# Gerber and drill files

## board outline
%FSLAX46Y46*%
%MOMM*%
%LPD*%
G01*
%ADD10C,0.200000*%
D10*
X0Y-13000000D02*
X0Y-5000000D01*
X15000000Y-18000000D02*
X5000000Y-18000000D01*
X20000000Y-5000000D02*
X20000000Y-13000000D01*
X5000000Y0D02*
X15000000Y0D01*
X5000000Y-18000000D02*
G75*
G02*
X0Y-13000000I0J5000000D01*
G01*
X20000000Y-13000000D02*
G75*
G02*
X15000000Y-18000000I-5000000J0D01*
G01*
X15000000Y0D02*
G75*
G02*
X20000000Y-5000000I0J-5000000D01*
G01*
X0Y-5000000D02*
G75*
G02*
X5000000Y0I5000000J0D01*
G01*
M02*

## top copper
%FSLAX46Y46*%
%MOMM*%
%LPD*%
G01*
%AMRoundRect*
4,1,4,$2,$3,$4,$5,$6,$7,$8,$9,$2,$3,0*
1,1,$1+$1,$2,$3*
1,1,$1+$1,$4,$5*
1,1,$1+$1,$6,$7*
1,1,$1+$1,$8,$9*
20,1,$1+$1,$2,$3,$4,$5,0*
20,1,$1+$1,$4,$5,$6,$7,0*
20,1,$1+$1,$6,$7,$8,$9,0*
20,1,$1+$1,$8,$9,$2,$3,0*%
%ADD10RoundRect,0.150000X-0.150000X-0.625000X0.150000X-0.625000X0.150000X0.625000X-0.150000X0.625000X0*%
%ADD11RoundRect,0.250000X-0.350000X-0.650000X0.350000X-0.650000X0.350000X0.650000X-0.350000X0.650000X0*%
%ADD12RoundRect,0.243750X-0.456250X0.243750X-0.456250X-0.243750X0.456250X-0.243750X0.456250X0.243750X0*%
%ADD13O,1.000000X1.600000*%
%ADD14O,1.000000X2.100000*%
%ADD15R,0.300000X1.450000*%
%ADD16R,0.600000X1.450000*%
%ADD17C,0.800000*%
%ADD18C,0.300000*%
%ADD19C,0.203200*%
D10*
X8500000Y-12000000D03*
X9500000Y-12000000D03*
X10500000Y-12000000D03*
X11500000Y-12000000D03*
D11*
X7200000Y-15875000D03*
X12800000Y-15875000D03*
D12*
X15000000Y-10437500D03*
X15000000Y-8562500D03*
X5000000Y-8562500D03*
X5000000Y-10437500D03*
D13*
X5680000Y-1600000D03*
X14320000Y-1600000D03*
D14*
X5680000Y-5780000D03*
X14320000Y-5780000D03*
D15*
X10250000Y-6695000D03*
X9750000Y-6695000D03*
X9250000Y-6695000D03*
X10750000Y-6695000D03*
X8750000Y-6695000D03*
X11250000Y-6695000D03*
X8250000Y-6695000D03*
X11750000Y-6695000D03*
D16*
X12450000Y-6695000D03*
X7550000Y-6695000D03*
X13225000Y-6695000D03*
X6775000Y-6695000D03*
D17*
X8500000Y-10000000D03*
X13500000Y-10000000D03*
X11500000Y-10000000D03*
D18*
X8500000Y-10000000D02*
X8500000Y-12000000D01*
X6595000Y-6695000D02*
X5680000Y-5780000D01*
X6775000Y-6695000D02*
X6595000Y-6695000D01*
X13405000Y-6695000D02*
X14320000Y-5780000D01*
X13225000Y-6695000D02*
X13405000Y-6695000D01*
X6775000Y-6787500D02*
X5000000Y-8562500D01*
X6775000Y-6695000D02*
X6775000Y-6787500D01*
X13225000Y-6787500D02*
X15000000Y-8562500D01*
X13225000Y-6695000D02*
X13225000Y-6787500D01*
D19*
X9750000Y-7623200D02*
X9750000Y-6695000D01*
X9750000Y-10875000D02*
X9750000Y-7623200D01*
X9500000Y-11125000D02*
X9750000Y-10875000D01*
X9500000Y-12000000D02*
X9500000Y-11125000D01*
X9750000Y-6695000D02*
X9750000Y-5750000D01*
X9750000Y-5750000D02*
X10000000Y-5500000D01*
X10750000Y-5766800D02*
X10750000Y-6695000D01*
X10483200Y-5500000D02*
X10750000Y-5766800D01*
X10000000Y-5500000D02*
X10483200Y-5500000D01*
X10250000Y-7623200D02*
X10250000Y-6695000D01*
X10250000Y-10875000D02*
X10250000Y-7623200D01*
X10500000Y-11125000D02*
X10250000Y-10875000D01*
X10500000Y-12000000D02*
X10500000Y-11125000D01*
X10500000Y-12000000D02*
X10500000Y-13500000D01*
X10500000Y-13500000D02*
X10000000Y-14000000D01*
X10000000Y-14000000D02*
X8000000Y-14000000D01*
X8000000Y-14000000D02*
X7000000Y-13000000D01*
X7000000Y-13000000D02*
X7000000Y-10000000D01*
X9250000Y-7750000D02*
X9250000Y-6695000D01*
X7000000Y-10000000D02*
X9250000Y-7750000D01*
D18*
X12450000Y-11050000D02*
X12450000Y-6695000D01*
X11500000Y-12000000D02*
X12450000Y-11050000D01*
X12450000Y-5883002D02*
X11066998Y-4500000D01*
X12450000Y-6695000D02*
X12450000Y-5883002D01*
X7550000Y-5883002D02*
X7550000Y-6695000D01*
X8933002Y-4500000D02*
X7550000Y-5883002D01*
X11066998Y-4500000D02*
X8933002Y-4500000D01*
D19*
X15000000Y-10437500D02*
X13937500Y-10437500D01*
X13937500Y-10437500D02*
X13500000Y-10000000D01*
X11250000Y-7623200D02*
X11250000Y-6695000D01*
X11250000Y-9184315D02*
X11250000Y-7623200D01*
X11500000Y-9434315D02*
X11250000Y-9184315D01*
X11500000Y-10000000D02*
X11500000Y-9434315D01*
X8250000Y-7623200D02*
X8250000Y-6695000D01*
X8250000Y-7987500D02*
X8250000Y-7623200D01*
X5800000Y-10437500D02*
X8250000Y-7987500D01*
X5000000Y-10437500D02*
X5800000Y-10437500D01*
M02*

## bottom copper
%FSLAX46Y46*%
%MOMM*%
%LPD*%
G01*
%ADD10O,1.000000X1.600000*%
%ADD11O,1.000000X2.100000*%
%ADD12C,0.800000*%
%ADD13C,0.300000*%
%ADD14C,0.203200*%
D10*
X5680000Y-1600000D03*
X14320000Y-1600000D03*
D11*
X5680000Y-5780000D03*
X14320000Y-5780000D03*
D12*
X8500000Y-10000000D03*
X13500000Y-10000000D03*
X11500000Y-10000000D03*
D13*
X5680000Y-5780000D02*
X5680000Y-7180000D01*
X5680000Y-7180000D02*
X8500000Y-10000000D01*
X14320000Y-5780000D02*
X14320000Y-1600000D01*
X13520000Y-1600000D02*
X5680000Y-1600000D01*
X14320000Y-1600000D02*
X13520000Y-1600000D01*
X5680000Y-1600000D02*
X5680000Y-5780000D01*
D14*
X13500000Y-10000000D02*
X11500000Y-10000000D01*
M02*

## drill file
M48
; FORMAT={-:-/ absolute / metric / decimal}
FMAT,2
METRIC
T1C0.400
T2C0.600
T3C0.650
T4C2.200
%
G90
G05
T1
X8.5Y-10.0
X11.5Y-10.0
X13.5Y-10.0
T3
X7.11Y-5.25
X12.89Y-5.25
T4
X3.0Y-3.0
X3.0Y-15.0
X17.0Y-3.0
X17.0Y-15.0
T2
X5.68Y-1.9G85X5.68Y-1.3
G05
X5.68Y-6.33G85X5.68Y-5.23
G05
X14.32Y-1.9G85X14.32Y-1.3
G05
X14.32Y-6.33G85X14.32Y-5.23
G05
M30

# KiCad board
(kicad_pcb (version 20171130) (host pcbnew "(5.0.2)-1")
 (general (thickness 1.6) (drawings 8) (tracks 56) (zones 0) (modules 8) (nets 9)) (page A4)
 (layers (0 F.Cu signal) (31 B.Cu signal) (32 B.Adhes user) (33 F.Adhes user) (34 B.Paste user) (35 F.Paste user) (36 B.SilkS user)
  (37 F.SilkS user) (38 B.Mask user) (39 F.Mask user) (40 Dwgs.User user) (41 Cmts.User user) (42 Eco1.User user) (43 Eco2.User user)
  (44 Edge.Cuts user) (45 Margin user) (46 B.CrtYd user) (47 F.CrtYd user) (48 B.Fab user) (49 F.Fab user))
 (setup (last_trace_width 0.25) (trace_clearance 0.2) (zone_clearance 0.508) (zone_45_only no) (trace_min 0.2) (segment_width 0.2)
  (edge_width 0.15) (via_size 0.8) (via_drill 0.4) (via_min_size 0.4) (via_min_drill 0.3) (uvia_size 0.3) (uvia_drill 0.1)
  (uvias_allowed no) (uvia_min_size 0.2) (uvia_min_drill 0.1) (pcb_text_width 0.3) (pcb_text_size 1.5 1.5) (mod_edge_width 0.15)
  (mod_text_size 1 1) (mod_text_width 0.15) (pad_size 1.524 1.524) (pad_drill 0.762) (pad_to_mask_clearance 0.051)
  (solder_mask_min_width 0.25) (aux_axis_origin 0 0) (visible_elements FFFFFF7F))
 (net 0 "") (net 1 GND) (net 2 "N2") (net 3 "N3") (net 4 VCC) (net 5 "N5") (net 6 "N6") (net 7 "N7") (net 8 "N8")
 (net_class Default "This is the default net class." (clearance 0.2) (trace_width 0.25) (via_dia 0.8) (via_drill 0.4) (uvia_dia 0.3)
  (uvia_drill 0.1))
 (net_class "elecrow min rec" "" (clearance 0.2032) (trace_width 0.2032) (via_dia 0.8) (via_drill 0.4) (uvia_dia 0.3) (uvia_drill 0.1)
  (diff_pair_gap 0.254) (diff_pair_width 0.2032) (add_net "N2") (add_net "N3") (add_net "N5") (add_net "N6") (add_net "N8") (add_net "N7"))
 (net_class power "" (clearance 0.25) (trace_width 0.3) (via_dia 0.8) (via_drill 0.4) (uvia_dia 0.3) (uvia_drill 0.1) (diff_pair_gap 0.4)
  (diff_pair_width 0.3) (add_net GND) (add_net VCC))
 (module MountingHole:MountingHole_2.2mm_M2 (layer F.Cu) (at 3 15)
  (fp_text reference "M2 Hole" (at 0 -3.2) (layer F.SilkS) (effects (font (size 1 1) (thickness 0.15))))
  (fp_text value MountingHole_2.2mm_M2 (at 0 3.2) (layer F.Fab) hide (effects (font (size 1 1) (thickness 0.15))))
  (pad 1 np_thru_hole circle (at 0 0) (size 2.2 2.2) (drill 2.2) (layers *.Cu *.Mask)))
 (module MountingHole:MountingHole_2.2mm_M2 (layer F.Cu) (at 17 15)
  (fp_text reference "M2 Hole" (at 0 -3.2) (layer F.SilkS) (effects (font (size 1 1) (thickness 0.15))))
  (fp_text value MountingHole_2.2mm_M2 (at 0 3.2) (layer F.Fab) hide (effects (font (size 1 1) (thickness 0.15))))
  (pad 1 np_thru_hole circle (at 0 0) (size 2.2 2.2) (drill 2.2) (layers *.Cu *.Mask)))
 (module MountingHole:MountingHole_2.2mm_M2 (layer F.Cu) (at 17 3)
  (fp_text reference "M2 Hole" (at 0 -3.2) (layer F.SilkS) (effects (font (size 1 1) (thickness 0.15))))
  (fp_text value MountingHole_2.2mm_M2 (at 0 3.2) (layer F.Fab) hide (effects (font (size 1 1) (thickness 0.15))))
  (pad 1 np_thru_hole circle (at 0 0) (size 2.2 2.2) (drill 2.2) (layers *.Cu *.Mask)))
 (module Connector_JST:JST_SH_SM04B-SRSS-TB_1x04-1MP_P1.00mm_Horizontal (layer F.Cu) (at 10 14)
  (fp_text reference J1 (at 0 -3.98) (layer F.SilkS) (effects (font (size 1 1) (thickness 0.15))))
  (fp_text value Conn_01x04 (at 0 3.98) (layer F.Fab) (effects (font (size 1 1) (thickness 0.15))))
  (pad 1 smd roundrect (at -1.5 -2) (size 0.6 1.55) (layers F.Cu F.Paste F.Mask) (roundrect_rratio 0.25) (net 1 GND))
  (pad 2 smd roundrect (at -0.5 -2) (size 0.6 1.55) (layers F.Cu F.Paste F.Mask) (roundrect_rratio 0.25) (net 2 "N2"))
  (pad 3 smd roundrect (at 0.5 -2) (size 0.6 1.55) (layers F.Cu F.Paste F.Mask) (roundrect_rratio 0.25) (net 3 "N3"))
  (pad 4 smd roundrect (at 1.5 -2) (size 0.6 1.55) (layers F.Cu F.Paste F.Mask) (roundrect_rratio 0.25) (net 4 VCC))
  (pad MP smd roundrect (at -2.8 1.875) (size 1.2 1.8) (layers F.Cu F.Paste F.Mask) (roundrect_rratio 0.208333))
  (pad MP smd roundrect (at 2.8 1.875) (size 1.2 1.8) (layers F.Cu F.Paste F.Mask) (roundrect_rratio 0.208333)))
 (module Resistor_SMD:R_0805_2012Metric (layer F.Cu) (at 15 9.5 270)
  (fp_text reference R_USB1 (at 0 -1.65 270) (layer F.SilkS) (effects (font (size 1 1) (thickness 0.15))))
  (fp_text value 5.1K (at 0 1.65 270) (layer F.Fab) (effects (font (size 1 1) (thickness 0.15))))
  (pad 2 smd roundrect (at 0.9375 0 270) (size 0.975 1.4) (layers F.Cu F.Paste F.Mask) (roundrect_rratio 0.25) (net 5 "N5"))
  (pad 1 smd roundrect (at -0.9375 0 270) (size 0.975 1.4) (layers F.Cu F.Paste F.Mask) (roundrect_rratio 0.25) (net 1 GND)))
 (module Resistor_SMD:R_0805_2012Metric (layer F.Cu) (at 5 9.5 270)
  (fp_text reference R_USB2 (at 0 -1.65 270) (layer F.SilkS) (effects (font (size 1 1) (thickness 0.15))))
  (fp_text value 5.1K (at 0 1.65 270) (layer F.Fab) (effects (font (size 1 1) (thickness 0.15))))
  (pad 1 smd roundrect (at -0.9375 0 270) (size 0.975 1.4) (layers F.Cu F.Paste F.Mask) (roundrect_rratio 0.25) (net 1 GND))
  (pad 2 smd roundrect (at 0.9375 0 270) (size 0.975 1.4) (layers F.Cu F.Paste F.Mask) (roundrect_rratio 0.25) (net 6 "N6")))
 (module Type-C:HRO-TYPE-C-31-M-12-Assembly (layer F.Cu) (at 10 -1 180)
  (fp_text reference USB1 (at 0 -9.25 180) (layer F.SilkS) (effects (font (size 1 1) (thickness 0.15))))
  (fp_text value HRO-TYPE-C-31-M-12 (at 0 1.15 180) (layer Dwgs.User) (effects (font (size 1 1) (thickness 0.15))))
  (pad 13 thru_hole oval (at 4.32 -2.6 180) (size 1 1.6) (drill oval 0.6 1.2) (layers *.Cu *.Mask) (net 1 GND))
  (pad 13 thru_hole oval (at -4.32 -2.6 180) (size 1 1.6) (drill oval 0.6 1.2) (layers *.Cu *.Mask) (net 1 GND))
  (pad 13 thru_hole oval (at 4.32 -6.78 180) (size 1 2.1) (drill oval 0.6 1.7) (layers *.Cu *.Mask) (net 1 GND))
  (pad 13 thru_hole oval (at -4.32 -6.78 180) (size 1 2.1) (drill oval 0.6 1.7) (layers *.Cu *.Mask) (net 1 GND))
  (pad "" np_thru_hole circle (at -2.89 -6.25 180) (size 0.65 0.65) (drill 0.65) (layers *.Cu *.Mask))
  (pad "" np_thru_hole circle (at 2.89 -6.25 180) (size 0.65 0.65) (drill 0.65) (layers *.Cu *.Mask))
  (pad 6 smd rect (at -0.25 -7.695 180) (size 0.3 1.45) (layers F.Cu F.Paste F.Mask) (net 3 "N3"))
  (pad 7 smd rect (at 0.25 -7.695 180) (size 0.3 1.45) (layers F.Cu F.Paste F.Mask) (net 2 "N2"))
  (pad 8 smd rect (at 0.75 -7.695 180) (size 0.3 1.45) (layers F.Cu F.Paste F.Mask) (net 3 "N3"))
  (pad 5 smd rect (at -0.75 -7.695 180) (size 0.3 1.45) (layers F.Cu F.Paste F.Mask) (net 2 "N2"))
  (pad 9 smd rect (at 1.25 -7.695 180) (size 0.3 1.45) (layers F.Cu F.Paste F.Mask) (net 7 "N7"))
  (pad 4 smd rect (at -1.25 -7.695 180) (size 0.3 1.45) (layers F.Cu F.Paste F.Mask) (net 5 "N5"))
  (pad 10 smd rect (at 1.75 -7.695 180) (size 0.3 1.45) (layers F.Cu F.Paste F.Mask) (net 6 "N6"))
  (pad 3 smd rect (at -1.75 -7.695 180) (size 0.3 1.45) (layers F.Cu F.Paste F.Mask) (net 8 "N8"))
  (pad 2 smd rect (at -2.45 -7.695 180) (size 0.6 1.45) (layers F.Cu F.Paste F.Mask) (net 4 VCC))
  (pad 11 smd rect (at 2.45 -7.695 180) (size 0.6 1.45) (layers F.Cu F.Paste F.Mask) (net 4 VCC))
  (pad 1 smd rect (at -3.225 -7.695 180) (size 0.6 1.45) (layers F.Cu F.Paste F.Mask) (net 1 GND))
  (pad 12 smd rect (at 3.225 -7.695 180) (size 0.6 1.45) (layers F.Cu F.Paste F.Mask) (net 1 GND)))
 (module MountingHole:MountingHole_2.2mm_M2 (layer F.Cu) (at 3 3)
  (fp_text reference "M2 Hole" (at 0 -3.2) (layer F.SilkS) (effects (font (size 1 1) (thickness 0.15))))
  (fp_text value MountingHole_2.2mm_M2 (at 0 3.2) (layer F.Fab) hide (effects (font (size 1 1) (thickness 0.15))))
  (pad 1 np_thru_hole circle (at 0 0) (size 2.2 2.2) (drill 2.2) (layers *.Cu *.Mask)))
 (gr_line (start 0 13) (end 0 5) (layer Edge.Cuts) (width 0.2))
 (gr_line (start 15 18) (end 5 18) (layer Edge.Cuts) (width 0.2))
 (gr_line (start 20 5) (end 20 13) (layer Edge.Cuts) (width 0.2))
 (gr_line (start 5 0) (end 15 0) (layer Edge.Cuts) (width 0.2))
 (gr_arc (start 5 13) (end 0 13) (angle -90) (layer Edge.Cuts) (width 0.2))
 (gr_arc (start 15 13) (end 15 18) (angle -90) (layer Edge.Cuts) (width 0.2))
 (gr_arc (start 15 5) (end 20 5) (angle -90) (layer Edge.Cuts) (width 0.2))
 (gr_arc (start 5 5) (end 5 0) (angle -90) (layer Edge.Cuts) (width 0.2))
 (via (at 8.5 10) (size 0.8) (drill 0.4) (layers F.Cu B.Cu) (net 1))
 (segment (start 5.68 5.78) (end 5.68 7.18) (width 0.3) (layer B.Cu) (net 1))
 (segment (start 5.68 7.18) (end 8.5 10) (width 0.3) (layer B.Cu) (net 1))
 (segment (start 8.5 10) (end 8.5 12) (width 0.3) (layer F.Cu) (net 1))
 (segment (start 6.595 6.695) (end 5.68 5.78) (width 0.3) (layer F.Cu) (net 1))
 (segment (start 6.775 6.695) (end 6.595 6.695) (width 0.3) (layer F.Cu) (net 1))
 (segment (start 13.405 6.695) (end 14.32 5.78) (width 0.3) (layer F.Cu) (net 1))
 (segment (start 13.225 6.695) (end 13.405 6.695) (width 0.3) (layer F.Cu) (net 1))
 (segment (start 14.32 5.78) (end 14.32 1.6) (width 0.3) (layer B.Cu) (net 1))
 (segment (start 13.52 1.6) (end 5.68 1.6) (width 0.3) (layer B.Cu) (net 1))
 (segment (start 14.32 1.6) (end 13.52 1.6) (width 0.3) (layer B.Cu) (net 1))
 (segment (start 5.68 1.6) (end 5.68 5.78) (width 0.3) (layer B.Cu) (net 1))
 (segment (start 6.775 6.7875) (end 5 8.5625) (width 0.3) (layer F.Cu) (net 1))
 (segment (start 6.775 6.695) (end 6.775 6.7875) (width 0.3) (layer F.Cu) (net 1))
 (segment (start 13.225 6.7875) (end 15 8.5625) (width 0.3) (layer F.Cu) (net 1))
 (segment (start 13.225 6.695) (end 13.225 6.7875) (width 0.3) (layer F.Cu) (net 1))
 (segment (start 9.75 7.6232) (end 9.75 6.695) (width 0.2032) (layer F.Cu) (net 2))
 (segment (start 9.75 10.875) (end 9.75 7.6232) (width 0.2032) (layer F.Cu) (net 2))
 (segment (start 9.5 11.125) (end 9.75 10.875) (width 0.2032) (layer F.Cu) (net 2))
 (segment (start 9.5 12) (end 9.5 11.125) (width 0.2032) (layer F.Cu) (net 2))
 (segment (start 9.75 6.695) (end 9.75 5.75) (width 0.2032) (layer F.Cu) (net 2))
 (segment (start 9.75 5.75) (end 10 5.5) (width 0.2032) (layer F.Cu) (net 2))
 (segment (start 10.75 5.7668) (end 10.75 6.695) (width 0.2032) (layer F.Cu) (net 2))
 (segment (start 10.4832 5.5) (end 10.75 5.7668) (width 0.2032) (layer F.Cu) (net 2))
 (segment (start 10 5.5) (end 10.4832 5.5) (width 0.2032) (layer F.Cu) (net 2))
 (segment (start 10.25 7.6232) (end 10.25 6.695) (width 0.2032) (layer F.Cu) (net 3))
 (segment (start 10.25 10.875) (end 10.25 7.6232) (width 0.2032) (layer F.Cu) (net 3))
 (segment (start 10.5 11.125) (end 10.25 10.875) (width 0.2032) (layer F.Cu) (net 3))
 (segment (start 10.5 12) (end 10.5 11.125) (width 0.2032) (layer F.Cu) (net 3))
 (segment (start 10.5 12) (end 10.5 13.5) (width 0.2032) (layer F.Cu) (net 3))
 (segment (start 10.5 13.5) (end 10 14) (width 0.2032) (layer F.Cu) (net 3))
 (segment (start 10 14) (end 8 14) (width 0.2032) (layer F.Cu) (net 3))
 (segment (start 8 14) (end 7 13) (width 0.2032) (layer F.Cu) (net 3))
 (segment (start 7 13) (end 7 10) (width 0.2032) (layer F.Cu) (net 3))
 (segment (start 9.25 7.75) (end 9.25 6.695) (width 0.2032) (layer F.Cu) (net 3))
 (segment (start 7 10) (end 9.25 7.75) (width 0.2032) (layer F.Cu) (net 3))
 (segment (start 12.45 11.05) (end 12.45 6.695) (width 0.3) (layer F.Cu) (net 4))
 (segment (start 11.5 12) (end 12.45 11.05) (width 0.3) (layer F.Cu) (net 4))
 (segment (start 12.45 5.883002) (end 11.066998 4.5) (width 0.3) (layer F.Cu) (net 4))
 (segment (start 12.45 6.695) (end 12.45 5.883002) (width 0.3) (layer F.Cu) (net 4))
 (segment (start 7.55 5.883002) (end 7.55 6.695) (width 0.3) (layer F.Cu) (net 4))
 (segment (start 8.933002 4.5) (end 7.55 5.883002) (width 0.3) (layer F.Cu) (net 4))
 (segment (start 11.066998 4.5) (end 8.933002 4.5) (width 0.3) (layer F.Cu) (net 4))
 (via (at 13.5 10) (size 0.8) (drill 0.4) (layers F.Cu B.Cu) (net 5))
 (segment (start 15 10.4375) (end 13.9375 10.4375) (width 0.2032) (layer F.Cu) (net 5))
 (segment (start 13.9375 10.4375) (end 13.5 10) (width 0.2032) (layer F.Cu) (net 5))
 (via (at 11.5 10) (size 0.8) (drill 0.4) (layers F.Cu B.Cu) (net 5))
 (segment (start 13.5 10) (end 11.5 10) (width 0.2032) (layer B.Cu) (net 5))
 (segment (start 11.25 7.6232) (end 11.25 6.695) (width 0.2032) (layer F.Cu) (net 5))
 (segment (start 11.25 9.184315) (end 11.25 7.6232) (width 0.2032) (layer F.Cu) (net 5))
 (segment (start 11.5 9.434315) (end 11.25 9.184315) (width 0.2032) (layer F.Cu) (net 5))
 (segment (start 11.5 10) (end 11.5 9.434315) (width 0.2032) (layer F.Cu) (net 5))
 (segment (start 8.25 7.6232) (end 8.25 6.695) (width 0.2032) (layer F.Cu) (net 6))
 (segment (start 8.25 7.9875) (end 8.25 7.6232) (width 0.2032) (layer F.Cu) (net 6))
 (segment (start 5.8 10.4375) (end 8.25 7.9875) (width 0.2032) (layer F.Cu) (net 6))
 (segment (start 5 10.4375) (end 5.8 10.4375) (width 0.2032) (layer F.Cu) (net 6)))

